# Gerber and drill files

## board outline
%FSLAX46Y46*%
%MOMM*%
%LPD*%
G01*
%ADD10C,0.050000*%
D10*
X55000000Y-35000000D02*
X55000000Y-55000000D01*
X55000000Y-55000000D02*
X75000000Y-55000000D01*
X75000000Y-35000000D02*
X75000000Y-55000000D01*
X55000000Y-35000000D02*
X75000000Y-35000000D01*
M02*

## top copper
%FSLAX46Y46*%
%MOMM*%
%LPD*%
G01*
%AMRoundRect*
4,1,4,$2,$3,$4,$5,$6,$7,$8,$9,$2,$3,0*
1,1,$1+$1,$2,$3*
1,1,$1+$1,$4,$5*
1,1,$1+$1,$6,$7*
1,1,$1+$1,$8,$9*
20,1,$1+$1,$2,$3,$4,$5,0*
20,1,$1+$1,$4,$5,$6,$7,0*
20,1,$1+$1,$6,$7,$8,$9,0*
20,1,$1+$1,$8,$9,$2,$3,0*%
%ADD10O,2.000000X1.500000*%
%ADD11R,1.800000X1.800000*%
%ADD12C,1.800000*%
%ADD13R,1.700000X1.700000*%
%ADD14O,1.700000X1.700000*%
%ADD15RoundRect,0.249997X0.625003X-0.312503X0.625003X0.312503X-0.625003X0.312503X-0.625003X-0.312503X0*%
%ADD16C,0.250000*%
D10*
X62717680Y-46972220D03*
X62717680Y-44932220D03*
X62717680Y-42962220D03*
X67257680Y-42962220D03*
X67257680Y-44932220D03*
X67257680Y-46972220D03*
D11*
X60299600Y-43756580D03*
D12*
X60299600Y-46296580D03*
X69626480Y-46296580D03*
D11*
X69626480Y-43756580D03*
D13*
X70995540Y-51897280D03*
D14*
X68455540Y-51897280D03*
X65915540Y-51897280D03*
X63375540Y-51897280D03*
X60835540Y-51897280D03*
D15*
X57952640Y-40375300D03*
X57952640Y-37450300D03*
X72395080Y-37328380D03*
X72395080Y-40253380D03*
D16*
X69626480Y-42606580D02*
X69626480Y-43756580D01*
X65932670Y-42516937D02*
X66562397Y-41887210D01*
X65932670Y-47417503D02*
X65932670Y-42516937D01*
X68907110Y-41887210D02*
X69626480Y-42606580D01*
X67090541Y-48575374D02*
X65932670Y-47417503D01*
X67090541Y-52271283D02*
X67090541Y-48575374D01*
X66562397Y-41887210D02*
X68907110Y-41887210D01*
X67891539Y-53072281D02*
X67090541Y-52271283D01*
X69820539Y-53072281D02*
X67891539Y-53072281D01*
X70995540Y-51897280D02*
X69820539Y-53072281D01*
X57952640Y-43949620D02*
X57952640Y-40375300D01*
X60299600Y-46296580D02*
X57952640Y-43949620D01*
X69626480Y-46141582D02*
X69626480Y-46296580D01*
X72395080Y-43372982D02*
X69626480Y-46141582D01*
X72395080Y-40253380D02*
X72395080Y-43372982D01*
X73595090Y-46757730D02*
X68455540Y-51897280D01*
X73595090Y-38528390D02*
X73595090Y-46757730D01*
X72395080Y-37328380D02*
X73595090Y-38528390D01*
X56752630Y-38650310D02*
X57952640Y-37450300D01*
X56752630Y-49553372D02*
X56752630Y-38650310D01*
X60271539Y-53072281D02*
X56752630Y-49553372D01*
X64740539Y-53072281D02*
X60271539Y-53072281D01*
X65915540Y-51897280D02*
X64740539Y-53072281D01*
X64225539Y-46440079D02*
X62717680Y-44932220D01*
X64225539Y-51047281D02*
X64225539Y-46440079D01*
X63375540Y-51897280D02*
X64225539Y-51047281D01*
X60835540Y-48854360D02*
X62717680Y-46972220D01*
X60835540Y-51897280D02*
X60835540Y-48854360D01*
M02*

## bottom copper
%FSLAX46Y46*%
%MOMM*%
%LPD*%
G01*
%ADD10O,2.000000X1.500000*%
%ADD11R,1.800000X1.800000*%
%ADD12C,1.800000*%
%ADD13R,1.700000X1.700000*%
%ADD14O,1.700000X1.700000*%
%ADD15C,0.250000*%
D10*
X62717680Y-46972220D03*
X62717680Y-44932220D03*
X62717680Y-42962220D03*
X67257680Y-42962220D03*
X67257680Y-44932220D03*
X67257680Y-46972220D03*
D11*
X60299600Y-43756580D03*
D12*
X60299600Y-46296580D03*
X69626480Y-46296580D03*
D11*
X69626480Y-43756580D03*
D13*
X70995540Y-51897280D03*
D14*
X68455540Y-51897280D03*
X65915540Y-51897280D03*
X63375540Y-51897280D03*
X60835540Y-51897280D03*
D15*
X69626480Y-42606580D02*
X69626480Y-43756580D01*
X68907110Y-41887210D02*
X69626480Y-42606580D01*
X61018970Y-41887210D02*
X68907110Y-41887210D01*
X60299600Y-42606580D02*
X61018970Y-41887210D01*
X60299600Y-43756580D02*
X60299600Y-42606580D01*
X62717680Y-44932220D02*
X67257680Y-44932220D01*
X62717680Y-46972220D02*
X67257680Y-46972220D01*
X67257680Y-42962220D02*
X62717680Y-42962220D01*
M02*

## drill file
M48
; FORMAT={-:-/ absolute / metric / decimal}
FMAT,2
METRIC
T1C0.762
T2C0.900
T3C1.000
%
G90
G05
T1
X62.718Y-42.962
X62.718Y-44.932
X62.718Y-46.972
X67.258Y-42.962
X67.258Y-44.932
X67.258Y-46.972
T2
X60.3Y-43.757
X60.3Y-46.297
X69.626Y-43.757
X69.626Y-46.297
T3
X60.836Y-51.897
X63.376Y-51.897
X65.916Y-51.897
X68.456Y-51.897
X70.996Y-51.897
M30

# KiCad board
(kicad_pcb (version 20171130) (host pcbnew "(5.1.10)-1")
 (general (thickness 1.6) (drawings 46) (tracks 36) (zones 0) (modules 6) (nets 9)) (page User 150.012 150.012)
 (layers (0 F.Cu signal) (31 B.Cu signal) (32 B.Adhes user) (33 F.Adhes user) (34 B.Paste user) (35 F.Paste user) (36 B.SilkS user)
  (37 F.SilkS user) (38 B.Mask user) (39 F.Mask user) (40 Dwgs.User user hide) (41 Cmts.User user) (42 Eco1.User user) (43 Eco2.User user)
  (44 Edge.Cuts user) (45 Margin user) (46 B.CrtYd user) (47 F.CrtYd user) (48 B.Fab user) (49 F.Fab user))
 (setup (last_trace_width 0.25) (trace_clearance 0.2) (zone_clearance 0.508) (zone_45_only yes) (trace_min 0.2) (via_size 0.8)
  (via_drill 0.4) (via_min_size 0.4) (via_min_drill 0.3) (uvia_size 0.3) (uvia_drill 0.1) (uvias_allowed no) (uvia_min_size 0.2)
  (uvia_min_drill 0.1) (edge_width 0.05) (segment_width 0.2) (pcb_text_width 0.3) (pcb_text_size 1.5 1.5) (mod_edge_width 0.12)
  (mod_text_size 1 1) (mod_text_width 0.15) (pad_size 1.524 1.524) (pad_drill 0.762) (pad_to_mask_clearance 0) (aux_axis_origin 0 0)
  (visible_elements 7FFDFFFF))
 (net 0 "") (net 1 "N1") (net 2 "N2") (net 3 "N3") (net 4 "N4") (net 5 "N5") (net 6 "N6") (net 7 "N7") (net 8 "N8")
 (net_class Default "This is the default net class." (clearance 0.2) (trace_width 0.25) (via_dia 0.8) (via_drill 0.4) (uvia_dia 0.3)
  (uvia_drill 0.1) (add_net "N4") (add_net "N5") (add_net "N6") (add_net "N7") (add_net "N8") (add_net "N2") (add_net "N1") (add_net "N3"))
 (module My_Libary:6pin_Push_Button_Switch (layer B.Cu) (at 70.33768 44.43222 90)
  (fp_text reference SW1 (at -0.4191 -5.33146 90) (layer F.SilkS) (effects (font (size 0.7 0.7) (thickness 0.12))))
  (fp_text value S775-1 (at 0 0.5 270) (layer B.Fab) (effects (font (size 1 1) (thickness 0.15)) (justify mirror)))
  (pad 1 thru_hole oval (at -2.54 -7.62 90) (size 1.5 2) (drill 0.762) (layers *.Cu *.Mask) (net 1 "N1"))
  (pad 2 thru_hole oval (at -0.5 -7.62 90) (size 1.5 2) (drill 0.762) (layers *.Cu *.Mask) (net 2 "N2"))
  (pad 3 thru_hole oval (at 1.47 -7.62 90) (size 1.5 2) (drill 0.762) (layers *.Cu *.Mask) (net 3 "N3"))
  (pad 3 thru_hole oval (at 1.47 -3.08 90) (size 1.5 2) (drill 0.762) (layers *.Cu *.Mask) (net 3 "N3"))
  (pad 2 thru_hole oval (at -0.5 -3.08 90) (size 1.5 2) (drill 0.762) (layers *.Cu *.Mask) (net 2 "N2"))
  (pad 1 thru_hole oval (at -2.54 -3.08 90) (size 1.5 2) (drill 0.762) (layers *.Cu *.Mask) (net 1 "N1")))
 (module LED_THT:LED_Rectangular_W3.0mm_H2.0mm (layer B.Cu) (at 60.2996 43.75658 270)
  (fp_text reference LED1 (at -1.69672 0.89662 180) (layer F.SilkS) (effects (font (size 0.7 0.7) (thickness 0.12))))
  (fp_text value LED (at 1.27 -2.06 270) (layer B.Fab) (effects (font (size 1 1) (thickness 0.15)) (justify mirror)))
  (pad 1 thru_hole rect (at 0 0 270) (size 1.8 1.8) (drill 0.9) (layers *.Cu *.Mask) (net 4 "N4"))
  (pad 2 thru_hole circle (at 2.54 0 270) (size 1.8 1.8) (drill 0.9) (layers *.Cu *.Mask) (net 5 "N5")))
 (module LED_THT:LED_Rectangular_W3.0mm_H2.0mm (layer B.Cu) (at 69.62648 43.75658 270)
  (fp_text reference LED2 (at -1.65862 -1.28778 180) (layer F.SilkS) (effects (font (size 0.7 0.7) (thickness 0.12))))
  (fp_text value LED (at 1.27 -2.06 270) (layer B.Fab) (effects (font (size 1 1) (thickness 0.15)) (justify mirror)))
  (pad 2 thru_hole circle (at 2.54 0 270) (size 1.8 1.8) (drill 0.9) (layers *.Cu *.Mask) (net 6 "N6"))
  (pad 1 thru_hole rect (at 0 0 270) (size 1.8 1.8) (drill 0.9) (layers *.Cu *.Mask) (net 4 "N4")))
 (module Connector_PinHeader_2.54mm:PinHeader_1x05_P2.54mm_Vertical (layer F.Cu) (at 70.99554 51.89728 270)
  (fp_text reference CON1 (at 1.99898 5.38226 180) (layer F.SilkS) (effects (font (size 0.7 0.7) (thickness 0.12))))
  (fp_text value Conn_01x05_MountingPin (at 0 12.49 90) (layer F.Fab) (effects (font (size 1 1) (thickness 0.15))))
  (pad 1 thru_hole rect (at 0 0 270) (size 1.7 1.7) (drill 1) (layers *.Cu *.Mask) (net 4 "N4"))
  (pad 2 thru_hole oval (at 0 2.54 270) (size 1.7 1.7) (drill 1) (layers *.Cu *.Mask) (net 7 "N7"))
  (pad 3 thru_hole oval (at 0 5.08 270) (size 1.7 1.7) (drill 1) (layers *.Cu *.Mask) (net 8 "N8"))
  (pad 4 thru_hole oval (at 0 7.62 270) (size 1.7 1.7) (drill 1) (layers *.Cu *.Mask) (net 2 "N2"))
  (pad 5 thru_hole oval (at 0 10.16 270) (size 1.7 1.7) (drill 1) (layers *.Cu *.Mask) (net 1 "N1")))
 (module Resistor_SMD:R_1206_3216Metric (layer F.Cu) (at 57.95264 38.9128 90)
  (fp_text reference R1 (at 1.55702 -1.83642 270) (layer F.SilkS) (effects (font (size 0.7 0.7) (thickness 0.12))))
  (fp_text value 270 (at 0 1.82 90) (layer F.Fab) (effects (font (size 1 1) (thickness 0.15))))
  (pad 1 smd roundrect (at -1.4625 0 90) (size 1.125 1.75) (layers F.Cu F.Paste F.Mask) (roundrect_rratio 0.2222195555555556) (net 5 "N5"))
  (pad 2 smd roundrect (at 1.4625 0 90) (size 1.125 1.75) (layers F.Cu F.Paste F.Mask) (roundrect_rratio 0.2222195555555556) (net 8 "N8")))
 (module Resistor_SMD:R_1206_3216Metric (layer F.Cu) (at 72.39508 38.79088 90)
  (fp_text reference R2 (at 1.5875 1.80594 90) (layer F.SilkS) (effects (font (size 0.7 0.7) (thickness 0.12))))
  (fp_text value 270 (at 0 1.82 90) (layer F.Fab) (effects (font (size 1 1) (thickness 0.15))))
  (pad 2 smd roundrect (at 1.4625 0 90) (size 1.125 1.75) (layers F.Cu F.Paste F.Mask) (roundrect_rratio 0.2222195555555556) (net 7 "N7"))
  (pad 1 smd roundrect (at -1.4625 0 90) (size 1.125 1.75) (layers F.Cu F.Paste F.Mask) (roundrect_rratio 0.2222195555555556) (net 6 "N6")))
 (gr_line (start 55 35) (end 55 55) (layer Edge.Cuts) (width 0.05))
 (gr_line (start 55 55) (end 75 55) (layer Edge.Cuts) (width 0.05))
 (gr_line (start 75 35) (end 75 55) (layer Edge.Cuts) (width 0.05))
 (gr_line (start 55 35) (end 75 35) (layer Edge.Cuts) (width 0.05))
 (segment (start 69.62648 42.60658) (end 69.62648 43.75658) (width 0.25) (layer B.Cu) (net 4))
 (segment (start 68.90711 41.88721) (end 69.62648 42.60658) (width 0.25) (layer B.Cu) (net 4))
 (segment (start 61.01897 41.88721) (end 68.90711 41.88721) (width 0.25) (layer B.Cu) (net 4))
 (segment (start 60.2996 42.60658) (end 61.01897 41.88721) (width 0.25) (layer B.Cu) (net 4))
 (segment (start 60.2996 43.75658) (end 60.2996 42.60658) (width 0.25) (layer B.Cu) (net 4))
 (segment (start 69.62648 42.60658) (end 69.62648 43.75658) (width 0.25) (layer F.Cu) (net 4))
 (segment (start 65.93267 42.516937) (end 66.562397 41.88721) (width 0.25) (layer F.Cu) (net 4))
 (segment (start 65.93267 47.417503) (end 65.93267 42.516937) (width 0.25) (layer F.Cu) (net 4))
 (segment (start 68.90711 41.88721) (end 69.62648 42.60658) (width 0.25) (layer F.Cu) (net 4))
 (segment (start 67.090541 48.575374) (end 65.93267 47.417503) (width 0.25) (layer F.Cu) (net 4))
 (segment (start 67.090541 52.271283) (end 67.090541 48.575374) (width 0.25) (layer F.Cu) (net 4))
 (segment (start 66.562397 41.88721) (end 68.90711 41.88721) (width 0.25) (layer F.Cu) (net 4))
 (segment (start 67.891539 53.072281) (end 67.090541 52.271283) (width 0.25) (layer F.Cu) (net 4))
 (segment (start 69.820539 53.072281) (end 67.891539 53.072281) (width 0.25) (layer F.Cu) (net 4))
 (segment (start 70.99554 51.89728) (end 69.820539 53.072281) (width 0.25) (layer F.Cu) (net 4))
 (segment (start 57.95264 43.94962) (end 57.95264 40.3753) (width 0.25) (layer F.Cu) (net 5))
 (segment (start 60.2996 46.29658) (end 57.95264 43.94962) (width 0.25) (layer F.Cu) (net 5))
 (segment (start 69.62648 46.141582) (end 69.62648 46.29658) (width 0.25) (layer F.Cu) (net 6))
 (segment (start 72.39508 43.372982) (end 69.62648 46.141582) (width 0.25) (layer F.Cu) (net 6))
 (segment (start 72.39508 40.25338) (end 72.39508 43.372982) (width 0.25) (layer F.Cu) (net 6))
 (segment (start 73.59509 46.75773) (end 68.45554 51.89728) (width 0.25) (layer F.Cu) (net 7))
 (segment (start 73.59509 38.52839) (end 73.59509 46.75773) (width 0.25) (layer F.Cu) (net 7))
 (segment (start 72.39508 37.32838) (end 73.59509 38.52839) (width 0.25) (layer F.Cu) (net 7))
 (segment (start 56.75263 38.65031) (end 57.95264 37.4503) (width 0.25) (layer F.Cu) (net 8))
 (segment (start 56.75263 49.553372) (end 56.75263 38.65031) (width 0.25) (layer F.Cu) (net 8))
 (segment (start 60.271539 53.072281) (end 56.75263 49.553372) (width 0.25) (layer F.Cu) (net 8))
 (segment (start 64.740539 53.072281) (end 60.271539 53.072281) (width 0.25) (layer F.Cu) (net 8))
 (segment (start 65.91554 51.89728) (end 64.740539 53.072281) (width 0.25) (layer F.Cu) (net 8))
 (segment (start 62.71768 44.93222) (end 67.25768 44.93222) (width 0.25) (layer B.Cu) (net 2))
 (segment (start 64.225539 46.440079) (end 62.71768 44.93222) (width 0.25) (layer F.Cu) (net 2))
 (segment (start 64.225539 51.047281) (end 64.225539 46.440079) (width 0.25) (layer F.Cu) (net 2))
 (segment (start 63.37554 51.89728) (end 64.225539 51.047281) (width 0.25) (layer F.Cu) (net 2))
 (segment (start 62.71768 46.97222) (end 67.25768 46.97222) (width 0.25) (layer B.Cu) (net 1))
 (segment (start 60.83554 48.85436) (end 62.71768 46.97222) (width 0.25) (layer F.Cu) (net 1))
 (segment (start 60.83554 51.89728) (end 60.83554 48.85436) (width 0.25) (layer F.Cu) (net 1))
 (segment (start 67.25768 42.96222) (end 62.71768 42.96222) (width 0.25) (layer B.Cu) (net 3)))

